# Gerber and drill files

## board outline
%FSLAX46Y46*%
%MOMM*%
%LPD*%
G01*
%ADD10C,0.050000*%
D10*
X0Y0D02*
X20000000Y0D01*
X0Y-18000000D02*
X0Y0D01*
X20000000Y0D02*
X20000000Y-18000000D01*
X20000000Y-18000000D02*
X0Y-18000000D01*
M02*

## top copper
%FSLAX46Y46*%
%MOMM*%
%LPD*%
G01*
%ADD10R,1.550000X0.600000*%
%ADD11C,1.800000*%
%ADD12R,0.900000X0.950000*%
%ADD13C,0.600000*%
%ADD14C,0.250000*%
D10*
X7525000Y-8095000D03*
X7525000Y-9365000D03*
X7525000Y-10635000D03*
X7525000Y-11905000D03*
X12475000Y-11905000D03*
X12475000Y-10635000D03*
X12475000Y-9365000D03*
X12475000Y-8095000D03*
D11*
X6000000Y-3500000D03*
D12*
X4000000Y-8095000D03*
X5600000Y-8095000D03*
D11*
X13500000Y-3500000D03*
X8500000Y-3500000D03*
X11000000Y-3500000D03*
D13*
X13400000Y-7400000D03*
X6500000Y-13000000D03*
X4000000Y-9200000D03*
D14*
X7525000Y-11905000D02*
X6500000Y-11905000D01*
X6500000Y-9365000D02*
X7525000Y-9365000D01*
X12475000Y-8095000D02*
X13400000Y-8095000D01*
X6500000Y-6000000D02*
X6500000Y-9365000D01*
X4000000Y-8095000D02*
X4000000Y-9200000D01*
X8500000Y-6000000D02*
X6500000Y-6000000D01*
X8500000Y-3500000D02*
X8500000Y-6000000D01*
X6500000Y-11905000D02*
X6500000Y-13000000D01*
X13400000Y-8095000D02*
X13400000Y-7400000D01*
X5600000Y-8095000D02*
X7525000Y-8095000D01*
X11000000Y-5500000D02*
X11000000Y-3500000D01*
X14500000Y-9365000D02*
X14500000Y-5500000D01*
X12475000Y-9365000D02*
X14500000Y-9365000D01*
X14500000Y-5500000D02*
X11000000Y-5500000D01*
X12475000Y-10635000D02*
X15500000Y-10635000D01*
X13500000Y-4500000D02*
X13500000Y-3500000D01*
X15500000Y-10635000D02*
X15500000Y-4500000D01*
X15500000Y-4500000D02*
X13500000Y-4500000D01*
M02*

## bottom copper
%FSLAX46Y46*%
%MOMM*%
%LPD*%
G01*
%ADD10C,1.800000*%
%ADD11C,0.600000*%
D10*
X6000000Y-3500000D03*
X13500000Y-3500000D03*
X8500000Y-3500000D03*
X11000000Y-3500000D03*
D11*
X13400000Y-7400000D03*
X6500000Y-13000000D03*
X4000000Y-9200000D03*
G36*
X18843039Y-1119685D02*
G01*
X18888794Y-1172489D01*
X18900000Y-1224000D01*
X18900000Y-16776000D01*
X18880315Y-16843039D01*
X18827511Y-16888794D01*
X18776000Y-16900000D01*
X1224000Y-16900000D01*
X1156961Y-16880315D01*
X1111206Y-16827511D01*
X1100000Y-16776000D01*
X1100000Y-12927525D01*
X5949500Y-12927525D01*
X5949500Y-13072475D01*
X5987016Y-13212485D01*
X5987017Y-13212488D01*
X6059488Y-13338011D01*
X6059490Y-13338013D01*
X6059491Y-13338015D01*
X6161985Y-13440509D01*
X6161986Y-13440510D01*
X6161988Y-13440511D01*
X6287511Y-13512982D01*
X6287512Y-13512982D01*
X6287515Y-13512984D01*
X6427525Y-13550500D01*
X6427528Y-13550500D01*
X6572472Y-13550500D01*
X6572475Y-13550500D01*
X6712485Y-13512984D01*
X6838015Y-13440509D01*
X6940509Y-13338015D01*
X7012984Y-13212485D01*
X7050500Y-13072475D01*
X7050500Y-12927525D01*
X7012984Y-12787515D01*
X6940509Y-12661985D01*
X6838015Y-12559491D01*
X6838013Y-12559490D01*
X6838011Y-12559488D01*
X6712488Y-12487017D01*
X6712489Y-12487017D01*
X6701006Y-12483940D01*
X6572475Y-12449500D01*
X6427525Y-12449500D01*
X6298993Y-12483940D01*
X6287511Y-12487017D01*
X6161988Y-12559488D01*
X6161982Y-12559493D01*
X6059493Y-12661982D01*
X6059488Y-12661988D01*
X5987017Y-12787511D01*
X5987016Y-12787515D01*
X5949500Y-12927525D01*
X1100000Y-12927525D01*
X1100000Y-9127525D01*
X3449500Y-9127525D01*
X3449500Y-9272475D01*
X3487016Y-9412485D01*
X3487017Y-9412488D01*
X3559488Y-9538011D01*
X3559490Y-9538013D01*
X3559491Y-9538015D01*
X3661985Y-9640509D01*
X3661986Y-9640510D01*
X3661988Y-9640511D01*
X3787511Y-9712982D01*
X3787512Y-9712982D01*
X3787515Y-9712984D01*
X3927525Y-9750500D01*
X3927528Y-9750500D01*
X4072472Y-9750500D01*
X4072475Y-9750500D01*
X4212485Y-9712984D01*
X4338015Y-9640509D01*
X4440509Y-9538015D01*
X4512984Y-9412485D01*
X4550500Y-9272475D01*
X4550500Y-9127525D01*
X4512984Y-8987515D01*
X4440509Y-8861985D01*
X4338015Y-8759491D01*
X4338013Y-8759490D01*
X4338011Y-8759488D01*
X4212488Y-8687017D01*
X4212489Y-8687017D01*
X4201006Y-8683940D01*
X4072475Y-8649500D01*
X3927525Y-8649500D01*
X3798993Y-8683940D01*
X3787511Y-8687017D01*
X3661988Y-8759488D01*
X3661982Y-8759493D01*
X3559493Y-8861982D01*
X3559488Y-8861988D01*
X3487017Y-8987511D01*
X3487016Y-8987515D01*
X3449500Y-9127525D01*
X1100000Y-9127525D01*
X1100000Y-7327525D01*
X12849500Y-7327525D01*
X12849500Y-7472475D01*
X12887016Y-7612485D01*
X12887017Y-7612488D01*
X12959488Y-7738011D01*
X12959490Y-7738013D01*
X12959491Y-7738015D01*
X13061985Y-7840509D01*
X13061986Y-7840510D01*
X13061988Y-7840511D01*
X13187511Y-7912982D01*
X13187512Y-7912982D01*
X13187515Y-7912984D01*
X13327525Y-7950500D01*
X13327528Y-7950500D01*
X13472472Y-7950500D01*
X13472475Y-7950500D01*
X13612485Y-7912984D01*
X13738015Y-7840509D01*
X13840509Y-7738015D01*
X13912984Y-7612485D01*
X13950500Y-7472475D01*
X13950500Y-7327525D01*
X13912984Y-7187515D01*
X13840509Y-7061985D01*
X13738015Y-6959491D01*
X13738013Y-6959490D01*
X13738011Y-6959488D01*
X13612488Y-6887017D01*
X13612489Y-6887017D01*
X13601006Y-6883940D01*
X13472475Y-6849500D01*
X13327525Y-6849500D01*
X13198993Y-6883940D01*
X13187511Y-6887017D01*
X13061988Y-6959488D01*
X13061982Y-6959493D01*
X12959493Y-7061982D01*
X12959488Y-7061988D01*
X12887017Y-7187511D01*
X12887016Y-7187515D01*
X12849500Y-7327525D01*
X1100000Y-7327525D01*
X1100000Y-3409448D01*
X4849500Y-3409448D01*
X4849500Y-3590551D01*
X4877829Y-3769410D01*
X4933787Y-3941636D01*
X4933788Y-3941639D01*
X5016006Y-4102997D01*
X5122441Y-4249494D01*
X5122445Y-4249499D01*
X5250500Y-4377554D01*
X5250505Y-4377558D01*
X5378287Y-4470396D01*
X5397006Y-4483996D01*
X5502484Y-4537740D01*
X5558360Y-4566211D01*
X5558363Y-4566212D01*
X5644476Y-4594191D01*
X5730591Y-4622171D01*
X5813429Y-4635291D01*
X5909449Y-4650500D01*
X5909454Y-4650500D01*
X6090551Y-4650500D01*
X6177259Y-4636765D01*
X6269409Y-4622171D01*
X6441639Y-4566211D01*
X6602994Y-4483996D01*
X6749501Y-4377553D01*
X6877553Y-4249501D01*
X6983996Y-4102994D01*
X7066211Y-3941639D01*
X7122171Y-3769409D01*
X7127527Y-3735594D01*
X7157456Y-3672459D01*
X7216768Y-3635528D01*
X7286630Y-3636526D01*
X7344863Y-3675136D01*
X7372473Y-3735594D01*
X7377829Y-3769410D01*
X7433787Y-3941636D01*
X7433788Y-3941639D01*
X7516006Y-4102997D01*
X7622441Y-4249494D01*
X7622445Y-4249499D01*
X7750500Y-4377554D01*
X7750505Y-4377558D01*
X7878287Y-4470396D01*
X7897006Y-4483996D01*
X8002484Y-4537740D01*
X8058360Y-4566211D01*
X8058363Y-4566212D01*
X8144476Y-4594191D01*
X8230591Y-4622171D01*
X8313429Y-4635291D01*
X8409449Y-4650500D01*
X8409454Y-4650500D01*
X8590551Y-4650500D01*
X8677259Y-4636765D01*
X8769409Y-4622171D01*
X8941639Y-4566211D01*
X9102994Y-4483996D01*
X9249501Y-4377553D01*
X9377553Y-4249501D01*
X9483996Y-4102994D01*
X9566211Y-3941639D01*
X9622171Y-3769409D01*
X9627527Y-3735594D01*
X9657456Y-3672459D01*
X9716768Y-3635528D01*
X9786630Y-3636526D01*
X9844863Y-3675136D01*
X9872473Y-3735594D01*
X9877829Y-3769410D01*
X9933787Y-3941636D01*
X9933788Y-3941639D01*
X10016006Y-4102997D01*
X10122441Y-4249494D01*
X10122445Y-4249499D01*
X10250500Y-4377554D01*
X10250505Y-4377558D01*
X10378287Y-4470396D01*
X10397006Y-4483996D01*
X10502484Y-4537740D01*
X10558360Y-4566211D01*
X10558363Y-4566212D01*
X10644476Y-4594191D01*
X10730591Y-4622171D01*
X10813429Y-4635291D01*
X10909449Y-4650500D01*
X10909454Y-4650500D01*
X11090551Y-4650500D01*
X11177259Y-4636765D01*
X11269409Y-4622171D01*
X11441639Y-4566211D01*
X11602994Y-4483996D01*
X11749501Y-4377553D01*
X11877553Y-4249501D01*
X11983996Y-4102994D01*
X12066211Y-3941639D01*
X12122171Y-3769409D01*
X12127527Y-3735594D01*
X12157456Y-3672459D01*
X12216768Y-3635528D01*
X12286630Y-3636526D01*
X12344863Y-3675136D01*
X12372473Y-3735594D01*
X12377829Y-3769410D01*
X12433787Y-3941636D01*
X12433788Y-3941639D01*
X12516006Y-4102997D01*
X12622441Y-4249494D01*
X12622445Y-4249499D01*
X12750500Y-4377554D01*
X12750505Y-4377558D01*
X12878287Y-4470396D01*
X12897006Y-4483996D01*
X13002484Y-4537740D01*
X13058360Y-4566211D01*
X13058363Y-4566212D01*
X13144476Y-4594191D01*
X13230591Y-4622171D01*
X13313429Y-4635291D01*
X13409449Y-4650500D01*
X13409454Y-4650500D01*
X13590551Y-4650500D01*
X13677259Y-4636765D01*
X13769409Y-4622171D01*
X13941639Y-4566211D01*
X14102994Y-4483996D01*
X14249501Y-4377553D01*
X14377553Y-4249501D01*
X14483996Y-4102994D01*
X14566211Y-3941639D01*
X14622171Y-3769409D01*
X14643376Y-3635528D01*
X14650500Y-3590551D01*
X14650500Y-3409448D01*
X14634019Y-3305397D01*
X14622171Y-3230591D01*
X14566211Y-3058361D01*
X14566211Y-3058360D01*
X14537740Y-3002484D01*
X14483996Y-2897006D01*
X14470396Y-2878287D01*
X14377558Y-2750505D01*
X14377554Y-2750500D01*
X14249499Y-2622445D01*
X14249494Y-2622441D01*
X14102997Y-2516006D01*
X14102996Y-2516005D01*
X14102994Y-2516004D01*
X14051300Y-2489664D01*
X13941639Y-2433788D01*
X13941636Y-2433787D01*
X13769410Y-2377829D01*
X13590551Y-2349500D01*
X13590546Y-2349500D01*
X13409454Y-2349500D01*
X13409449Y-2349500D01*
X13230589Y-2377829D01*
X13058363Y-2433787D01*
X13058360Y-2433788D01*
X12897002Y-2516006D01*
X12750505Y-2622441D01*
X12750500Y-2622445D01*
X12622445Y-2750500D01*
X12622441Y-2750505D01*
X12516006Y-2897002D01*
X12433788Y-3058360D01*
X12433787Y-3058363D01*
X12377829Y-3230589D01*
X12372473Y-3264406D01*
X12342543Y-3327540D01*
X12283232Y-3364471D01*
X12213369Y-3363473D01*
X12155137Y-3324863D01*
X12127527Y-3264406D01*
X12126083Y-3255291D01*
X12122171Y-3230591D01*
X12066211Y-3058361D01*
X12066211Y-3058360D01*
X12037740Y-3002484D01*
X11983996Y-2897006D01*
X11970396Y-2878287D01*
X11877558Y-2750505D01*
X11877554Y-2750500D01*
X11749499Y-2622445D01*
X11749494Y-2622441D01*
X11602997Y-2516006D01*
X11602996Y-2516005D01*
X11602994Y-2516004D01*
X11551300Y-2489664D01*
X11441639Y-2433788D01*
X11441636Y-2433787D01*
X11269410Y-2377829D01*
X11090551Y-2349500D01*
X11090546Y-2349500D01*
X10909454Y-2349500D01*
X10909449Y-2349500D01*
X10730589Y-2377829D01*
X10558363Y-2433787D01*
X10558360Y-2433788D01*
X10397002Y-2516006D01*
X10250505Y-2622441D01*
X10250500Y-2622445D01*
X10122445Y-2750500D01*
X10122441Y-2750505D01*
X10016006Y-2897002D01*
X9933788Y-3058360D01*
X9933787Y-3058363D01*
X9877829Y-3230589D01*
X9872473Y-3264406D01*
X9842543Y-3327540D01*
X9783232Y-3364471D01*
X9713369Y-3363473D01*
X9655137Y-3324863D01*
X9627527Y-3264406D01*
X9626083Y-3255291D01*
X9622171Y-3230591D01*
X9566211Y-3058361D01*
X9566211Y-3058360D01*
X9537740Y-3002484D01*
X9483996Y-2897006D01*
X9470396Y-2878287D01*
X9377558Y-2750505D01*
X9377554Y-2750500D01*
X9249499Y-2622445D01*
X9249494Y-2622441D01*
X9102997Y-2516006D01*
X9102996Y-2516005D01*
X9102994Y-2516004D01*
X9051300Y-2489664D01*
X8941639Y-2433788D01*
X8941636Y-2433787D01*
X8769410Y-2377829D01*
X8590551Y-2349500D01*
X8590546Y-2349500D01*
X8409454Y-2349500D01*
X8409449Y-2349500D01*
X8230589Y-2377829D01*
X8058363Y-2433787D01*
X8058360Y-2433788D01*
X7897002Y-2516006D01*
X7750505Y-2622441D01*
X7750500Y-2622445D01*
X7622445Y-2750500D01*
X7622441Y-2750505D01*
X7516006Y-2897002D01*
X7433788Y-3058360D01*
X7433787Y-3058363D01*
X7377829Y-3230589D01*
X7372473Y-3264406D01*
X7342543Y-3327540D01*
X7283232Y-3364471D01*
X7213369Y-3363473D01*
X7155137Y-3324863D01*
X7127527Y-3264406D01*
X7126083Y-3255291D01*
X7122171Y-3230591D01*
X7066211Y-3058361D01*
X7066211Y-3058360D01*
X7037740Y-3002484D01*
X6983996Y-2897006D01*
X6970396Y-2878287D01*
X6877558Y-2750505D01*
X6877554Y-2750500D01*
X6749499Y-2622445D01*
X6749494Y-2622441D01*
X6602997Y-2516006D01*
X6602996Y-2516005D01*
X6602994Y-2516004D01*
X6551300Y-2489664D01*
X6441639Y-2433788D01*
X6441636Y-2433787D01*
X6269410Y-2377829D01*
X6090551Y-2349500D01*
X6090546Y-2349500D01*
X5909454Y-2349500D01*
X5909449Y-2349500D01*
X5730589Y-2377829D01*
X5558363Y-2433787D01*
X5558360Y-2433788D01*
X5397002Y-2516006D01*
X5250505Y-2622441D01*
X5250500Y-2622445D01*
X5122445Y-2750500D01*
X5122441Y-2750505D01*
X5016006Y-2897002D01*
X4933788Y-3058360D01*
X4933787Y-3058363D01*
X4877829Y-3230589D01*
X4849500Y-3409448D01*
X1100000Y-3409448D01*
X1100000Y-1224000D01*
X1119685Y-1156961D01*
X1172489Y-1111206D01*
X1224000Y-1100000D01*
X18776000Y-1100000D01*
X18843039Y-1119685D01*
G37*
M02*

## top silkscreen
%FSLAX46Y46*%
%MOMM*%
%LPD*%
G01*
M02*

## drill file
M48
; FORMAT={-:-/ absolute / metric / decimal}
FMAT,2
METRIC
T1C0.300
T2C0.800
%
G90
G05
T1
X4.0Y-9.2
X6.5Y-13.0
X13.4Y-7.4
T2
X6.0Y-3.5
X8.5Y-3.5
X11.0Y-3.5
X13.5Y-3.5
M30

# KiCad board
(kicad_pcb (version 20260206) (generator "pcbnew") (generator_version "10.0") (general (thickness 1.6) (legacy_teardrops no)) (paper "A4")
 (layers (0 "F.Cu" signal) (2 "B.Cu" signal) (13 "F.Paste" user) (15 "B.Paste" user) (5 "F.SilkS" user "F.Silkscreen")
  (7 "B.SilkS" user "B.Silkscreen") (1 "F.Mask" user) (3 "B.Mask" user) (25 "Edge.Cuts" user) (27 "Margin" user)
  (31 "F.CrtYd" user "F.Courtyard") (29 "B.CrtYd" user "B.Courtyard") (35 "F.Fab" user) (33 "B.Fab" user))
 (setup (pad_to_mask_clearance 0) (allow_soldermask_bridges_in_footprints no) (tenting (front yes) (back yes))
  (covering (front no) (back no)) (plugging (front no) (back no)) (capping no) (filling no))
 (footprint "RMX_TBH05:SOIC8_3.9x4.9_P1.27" (layer "F.Cu") (at 10 10)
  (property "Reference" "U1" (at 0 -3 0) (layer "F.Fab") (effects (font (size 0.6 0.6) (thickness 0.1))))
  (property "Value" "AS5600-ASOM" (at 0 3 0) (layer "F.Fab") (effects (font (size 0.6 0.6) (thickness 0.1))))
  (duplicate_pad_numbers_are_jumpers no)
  (pad "1" smd rect (at -2.475 -1.905) (size 1.55 0.6) (layers "F.Cu" "F.Mask" "F.Paste") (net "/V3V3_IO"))
  (pad "2" smd rect (at -2.475 -0.635) (size 1.55 0.6) (layers "F.Cu" "F.Mask" "F.Paste") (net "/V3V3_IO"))
  (pad "3" smd rect (at -2.475 0.635) (size 1.55 0.6) (layers "F.Cu" "F.Mask" "F.Paste") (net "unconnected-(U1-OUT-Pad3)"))
  (pad "4" smd rect (at -2.475 1.905) (size 1.55 0.6) (layers "F.Cu" "F.Mask" "F.Paste"))
  (pad "5" smd rect (at 2.475 1.905) (size 1.55 0.6) (layers "F.Cu" "F.Mask" "F.Paste") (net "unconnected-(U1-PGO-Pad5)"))
  (pad "6" smd rect (at 2.475 0.635) (size 1.55 0.6) (layers "F.Cu" "F.Mask" "F.Paste"))
  (pad "7" smd rect (at 2.475 -0.635) (size 1.55 0.6) (layers "F.Cu" "F.Mask" "F.Paste"))
  (pad "8" smd rect (at 2.475 -1.905) (size 1.55 0.6) (layers "F.Cu" "F.Mask" "F.Paste")))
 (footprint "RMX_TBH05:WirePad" (layer "F.Cu") (at 6 3.5)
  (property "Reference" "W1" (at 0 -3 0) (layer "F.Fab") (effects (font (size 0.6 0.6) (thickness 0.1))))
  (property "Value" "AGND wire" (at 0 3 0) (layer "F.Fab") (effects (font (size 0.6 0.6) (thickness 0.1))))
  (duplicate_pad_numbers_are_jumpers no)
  (pad "1" thru_hole circle (at 0 0) (size 1.8 1.8) (drill 0.8) (layers "*.Cu" "*.Mask") (remove_unused_layers no)))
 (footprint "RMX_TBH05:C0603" (layer "F.Cu") (at 4.8 8.095)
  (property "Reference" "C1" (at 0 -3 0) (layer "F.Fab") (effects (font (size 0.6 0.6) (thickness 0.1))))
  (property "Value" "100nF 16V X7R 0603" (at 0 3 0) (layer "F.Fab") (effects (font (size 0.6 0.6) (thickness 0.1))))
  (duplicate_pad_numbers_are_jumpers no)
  (pad "1" smd rect (at -0.8 0) (size 0.9 0.95) (layers "F.Cu" "F.Mask" "F.Paste"))
  (pad "2" smd rect (at 0.8 0) (size 0.9 0.95) (layers "F.Cu" "F.Mask" "F.Paste") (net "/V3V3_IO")))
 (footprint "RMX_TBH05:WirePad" (layer "F.Cu") (at 13.5 3.5)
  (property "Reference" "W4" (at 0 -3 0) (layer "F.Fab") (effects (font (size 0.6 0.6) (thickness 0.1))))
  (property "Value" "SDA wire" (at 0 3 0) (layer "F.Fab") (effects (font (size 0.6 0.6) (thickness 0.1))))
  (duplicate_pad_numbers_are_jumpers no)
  (pad "1" thru_hole circle (at 0 0) (size 1.8 1.8) (drill 0.8) (layers "*.Cu" "*.Mask") (remove_unused_layers no)))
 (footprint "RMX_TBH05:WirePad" (layer "F.Cu") (at 8.5 3.5)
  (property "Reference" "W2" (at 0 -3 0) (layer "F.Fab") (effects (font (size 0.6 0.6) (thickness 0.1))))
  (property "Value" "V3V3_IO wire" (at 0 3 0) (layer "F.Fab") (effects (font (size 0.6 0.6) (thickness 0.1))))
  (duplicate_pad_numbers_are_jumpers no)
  (pad "1" thru_hole circle (at 0 0) (size 1.8 1.8) (drill 0.8) (layers "*.Cu" "*.Mask") (remove_unused_layers no) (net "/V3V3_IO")))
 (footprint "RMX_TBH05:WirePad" (layer "F.Cu") (at 11 3.5)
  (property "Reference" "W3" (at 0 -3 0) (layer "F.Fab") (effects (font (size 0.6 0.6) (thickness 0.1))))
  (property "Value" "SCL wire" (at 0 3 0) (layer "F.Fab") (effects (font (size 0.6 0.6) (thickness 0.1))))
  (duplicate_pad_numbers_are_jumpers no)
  (pad "1" thru_hole circle (at 0 0) (size 1.8 1.8) (drill 0.8) (layers "*.Cu" "*.Mask") (remove_unused_layers no)))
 (gr_line (start 0 0) (end 20 0) (stroke (width 0.05) (type default)) (layer "Edge.Cuts"))
 (gr_line (start 0 18) (end 0 0) (stroke (width 0.05) (type default)) (layer "Edge.Cuts"))
 (gr_line (start 20 0) (end 20 18) (stroke (width 0.05) (type default)) (layer "Edge.Cuts"))
 (gr_line (start 20 18) (end 0 18) (stroke (width 0.05) (type default)) (layer "Edge.Cuts"))
 (segment (start 7.525 11.905) (end 6.5 11.905) (width 0.25) (layer "F.Cu") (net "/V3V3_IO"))
 (segment (start 6.5 9.365) (end 7.525 9.365) (width 0.25) (layer "F.Cu") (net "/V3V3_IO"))
 (segment (start 12.475 8.095) (end 13.4 8.095) (width 0.25) (layer "F.Cu") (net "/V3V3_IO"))
 (segment (start 6.5 6) (end 6.5 9.365) (width 0.25) (layer "F.Cu") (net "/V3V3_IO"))
 (segment (start 4 8.095) (end 4 9.2) (width 0.25) (layer "F.Cu") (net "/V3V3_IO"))
 (segment (start 8.5 6) (end 6.5 6) (width 0.25) (layer "F.Cu") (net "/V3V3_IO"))
 (segment (start 8.5 3.5) (end 8.5 6) (width 0.25) (layer "F.Cu") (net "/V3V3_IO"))
 (segment (start 6.5 11.905) (end 6.5 13) (width 0.25) (layer "F.Cu") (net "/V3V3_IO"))
 (segment (start 13.4 8.095) (end 13.4 7.4) (width 0.25) (layer "F.Cu") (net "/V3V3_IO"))
 (segment (start 5.6 8.095) (end 7.525 8.095) (width 0.25) (layer "F.Cu") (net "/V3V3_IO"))
 (via (at 13.4 7.4) (size 0.6) (drill 0.3) (layers "F.Cu" "B.Cu") (capping no) (covering (front no) (back no))
  (plugging (front no) (back no)) (filling no) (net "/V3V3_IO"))
 (via (at 6.5 13) (size 0.6) (drill 0.3) (layers "F.Cu" "B.Cu") (capping no) (covering (front no) (back no)) (plugging (front no) (back no))
  (filling no) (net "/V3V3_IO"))
 (via (at 4 9.2) (size 0.6) (drill 0.3) (layers "F.Cu" "B.Cu") (capping no) (covering (front no) (back no)) (plugging (front no) (back no))
  (filling no) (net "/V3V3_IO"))
 (segment (start 11 5.5) (end 11 3.5) (width 0.25) (layer "F.Cu") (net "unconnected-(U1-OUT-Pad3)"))
 (segment (start 14.5 9.365) (end 14.5 5.5) (width 0.25) (layer "F.Cu") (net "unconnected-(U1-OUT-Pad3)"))
 (segment (start 12.475 9.365) (end 14.5 9.365) (width 0.25) (layer "F.Cu") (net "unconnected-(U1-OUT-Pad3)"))
 (segment (start 14.5 5.5) (end 11 5.5) (width 0.25) (layer "F.Cu") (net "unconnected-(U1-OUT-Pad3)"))
 (segment (start 12.475 10.635) (end 15.5 10.635) (width 0.25) (layer "F.Cu") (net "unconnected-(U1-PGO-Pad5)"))
 (segment (start 13.5 4.5) (end 13.5 3.5) (width 0.25) (layer "F.Cu") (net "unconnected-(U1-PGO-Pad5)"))
 (segment (start 15.5 10.635) (end 15.5 4.5) (width 0.25) (layer "F.Cu") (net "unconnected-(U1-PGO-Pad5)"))
 (segment (start 15.5 4.5) (end 13.5 4.5) (width 0.25) (layer "F.Cu") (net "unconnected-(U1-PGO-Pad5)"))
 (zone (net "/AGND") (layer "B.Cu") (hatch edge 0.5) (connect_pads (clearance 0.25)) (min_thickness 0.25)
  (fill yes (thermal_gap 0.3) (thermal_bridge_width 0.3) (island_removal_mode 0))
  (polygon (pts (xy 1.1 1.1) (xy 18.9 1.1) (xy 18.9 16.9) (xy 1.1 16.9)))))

